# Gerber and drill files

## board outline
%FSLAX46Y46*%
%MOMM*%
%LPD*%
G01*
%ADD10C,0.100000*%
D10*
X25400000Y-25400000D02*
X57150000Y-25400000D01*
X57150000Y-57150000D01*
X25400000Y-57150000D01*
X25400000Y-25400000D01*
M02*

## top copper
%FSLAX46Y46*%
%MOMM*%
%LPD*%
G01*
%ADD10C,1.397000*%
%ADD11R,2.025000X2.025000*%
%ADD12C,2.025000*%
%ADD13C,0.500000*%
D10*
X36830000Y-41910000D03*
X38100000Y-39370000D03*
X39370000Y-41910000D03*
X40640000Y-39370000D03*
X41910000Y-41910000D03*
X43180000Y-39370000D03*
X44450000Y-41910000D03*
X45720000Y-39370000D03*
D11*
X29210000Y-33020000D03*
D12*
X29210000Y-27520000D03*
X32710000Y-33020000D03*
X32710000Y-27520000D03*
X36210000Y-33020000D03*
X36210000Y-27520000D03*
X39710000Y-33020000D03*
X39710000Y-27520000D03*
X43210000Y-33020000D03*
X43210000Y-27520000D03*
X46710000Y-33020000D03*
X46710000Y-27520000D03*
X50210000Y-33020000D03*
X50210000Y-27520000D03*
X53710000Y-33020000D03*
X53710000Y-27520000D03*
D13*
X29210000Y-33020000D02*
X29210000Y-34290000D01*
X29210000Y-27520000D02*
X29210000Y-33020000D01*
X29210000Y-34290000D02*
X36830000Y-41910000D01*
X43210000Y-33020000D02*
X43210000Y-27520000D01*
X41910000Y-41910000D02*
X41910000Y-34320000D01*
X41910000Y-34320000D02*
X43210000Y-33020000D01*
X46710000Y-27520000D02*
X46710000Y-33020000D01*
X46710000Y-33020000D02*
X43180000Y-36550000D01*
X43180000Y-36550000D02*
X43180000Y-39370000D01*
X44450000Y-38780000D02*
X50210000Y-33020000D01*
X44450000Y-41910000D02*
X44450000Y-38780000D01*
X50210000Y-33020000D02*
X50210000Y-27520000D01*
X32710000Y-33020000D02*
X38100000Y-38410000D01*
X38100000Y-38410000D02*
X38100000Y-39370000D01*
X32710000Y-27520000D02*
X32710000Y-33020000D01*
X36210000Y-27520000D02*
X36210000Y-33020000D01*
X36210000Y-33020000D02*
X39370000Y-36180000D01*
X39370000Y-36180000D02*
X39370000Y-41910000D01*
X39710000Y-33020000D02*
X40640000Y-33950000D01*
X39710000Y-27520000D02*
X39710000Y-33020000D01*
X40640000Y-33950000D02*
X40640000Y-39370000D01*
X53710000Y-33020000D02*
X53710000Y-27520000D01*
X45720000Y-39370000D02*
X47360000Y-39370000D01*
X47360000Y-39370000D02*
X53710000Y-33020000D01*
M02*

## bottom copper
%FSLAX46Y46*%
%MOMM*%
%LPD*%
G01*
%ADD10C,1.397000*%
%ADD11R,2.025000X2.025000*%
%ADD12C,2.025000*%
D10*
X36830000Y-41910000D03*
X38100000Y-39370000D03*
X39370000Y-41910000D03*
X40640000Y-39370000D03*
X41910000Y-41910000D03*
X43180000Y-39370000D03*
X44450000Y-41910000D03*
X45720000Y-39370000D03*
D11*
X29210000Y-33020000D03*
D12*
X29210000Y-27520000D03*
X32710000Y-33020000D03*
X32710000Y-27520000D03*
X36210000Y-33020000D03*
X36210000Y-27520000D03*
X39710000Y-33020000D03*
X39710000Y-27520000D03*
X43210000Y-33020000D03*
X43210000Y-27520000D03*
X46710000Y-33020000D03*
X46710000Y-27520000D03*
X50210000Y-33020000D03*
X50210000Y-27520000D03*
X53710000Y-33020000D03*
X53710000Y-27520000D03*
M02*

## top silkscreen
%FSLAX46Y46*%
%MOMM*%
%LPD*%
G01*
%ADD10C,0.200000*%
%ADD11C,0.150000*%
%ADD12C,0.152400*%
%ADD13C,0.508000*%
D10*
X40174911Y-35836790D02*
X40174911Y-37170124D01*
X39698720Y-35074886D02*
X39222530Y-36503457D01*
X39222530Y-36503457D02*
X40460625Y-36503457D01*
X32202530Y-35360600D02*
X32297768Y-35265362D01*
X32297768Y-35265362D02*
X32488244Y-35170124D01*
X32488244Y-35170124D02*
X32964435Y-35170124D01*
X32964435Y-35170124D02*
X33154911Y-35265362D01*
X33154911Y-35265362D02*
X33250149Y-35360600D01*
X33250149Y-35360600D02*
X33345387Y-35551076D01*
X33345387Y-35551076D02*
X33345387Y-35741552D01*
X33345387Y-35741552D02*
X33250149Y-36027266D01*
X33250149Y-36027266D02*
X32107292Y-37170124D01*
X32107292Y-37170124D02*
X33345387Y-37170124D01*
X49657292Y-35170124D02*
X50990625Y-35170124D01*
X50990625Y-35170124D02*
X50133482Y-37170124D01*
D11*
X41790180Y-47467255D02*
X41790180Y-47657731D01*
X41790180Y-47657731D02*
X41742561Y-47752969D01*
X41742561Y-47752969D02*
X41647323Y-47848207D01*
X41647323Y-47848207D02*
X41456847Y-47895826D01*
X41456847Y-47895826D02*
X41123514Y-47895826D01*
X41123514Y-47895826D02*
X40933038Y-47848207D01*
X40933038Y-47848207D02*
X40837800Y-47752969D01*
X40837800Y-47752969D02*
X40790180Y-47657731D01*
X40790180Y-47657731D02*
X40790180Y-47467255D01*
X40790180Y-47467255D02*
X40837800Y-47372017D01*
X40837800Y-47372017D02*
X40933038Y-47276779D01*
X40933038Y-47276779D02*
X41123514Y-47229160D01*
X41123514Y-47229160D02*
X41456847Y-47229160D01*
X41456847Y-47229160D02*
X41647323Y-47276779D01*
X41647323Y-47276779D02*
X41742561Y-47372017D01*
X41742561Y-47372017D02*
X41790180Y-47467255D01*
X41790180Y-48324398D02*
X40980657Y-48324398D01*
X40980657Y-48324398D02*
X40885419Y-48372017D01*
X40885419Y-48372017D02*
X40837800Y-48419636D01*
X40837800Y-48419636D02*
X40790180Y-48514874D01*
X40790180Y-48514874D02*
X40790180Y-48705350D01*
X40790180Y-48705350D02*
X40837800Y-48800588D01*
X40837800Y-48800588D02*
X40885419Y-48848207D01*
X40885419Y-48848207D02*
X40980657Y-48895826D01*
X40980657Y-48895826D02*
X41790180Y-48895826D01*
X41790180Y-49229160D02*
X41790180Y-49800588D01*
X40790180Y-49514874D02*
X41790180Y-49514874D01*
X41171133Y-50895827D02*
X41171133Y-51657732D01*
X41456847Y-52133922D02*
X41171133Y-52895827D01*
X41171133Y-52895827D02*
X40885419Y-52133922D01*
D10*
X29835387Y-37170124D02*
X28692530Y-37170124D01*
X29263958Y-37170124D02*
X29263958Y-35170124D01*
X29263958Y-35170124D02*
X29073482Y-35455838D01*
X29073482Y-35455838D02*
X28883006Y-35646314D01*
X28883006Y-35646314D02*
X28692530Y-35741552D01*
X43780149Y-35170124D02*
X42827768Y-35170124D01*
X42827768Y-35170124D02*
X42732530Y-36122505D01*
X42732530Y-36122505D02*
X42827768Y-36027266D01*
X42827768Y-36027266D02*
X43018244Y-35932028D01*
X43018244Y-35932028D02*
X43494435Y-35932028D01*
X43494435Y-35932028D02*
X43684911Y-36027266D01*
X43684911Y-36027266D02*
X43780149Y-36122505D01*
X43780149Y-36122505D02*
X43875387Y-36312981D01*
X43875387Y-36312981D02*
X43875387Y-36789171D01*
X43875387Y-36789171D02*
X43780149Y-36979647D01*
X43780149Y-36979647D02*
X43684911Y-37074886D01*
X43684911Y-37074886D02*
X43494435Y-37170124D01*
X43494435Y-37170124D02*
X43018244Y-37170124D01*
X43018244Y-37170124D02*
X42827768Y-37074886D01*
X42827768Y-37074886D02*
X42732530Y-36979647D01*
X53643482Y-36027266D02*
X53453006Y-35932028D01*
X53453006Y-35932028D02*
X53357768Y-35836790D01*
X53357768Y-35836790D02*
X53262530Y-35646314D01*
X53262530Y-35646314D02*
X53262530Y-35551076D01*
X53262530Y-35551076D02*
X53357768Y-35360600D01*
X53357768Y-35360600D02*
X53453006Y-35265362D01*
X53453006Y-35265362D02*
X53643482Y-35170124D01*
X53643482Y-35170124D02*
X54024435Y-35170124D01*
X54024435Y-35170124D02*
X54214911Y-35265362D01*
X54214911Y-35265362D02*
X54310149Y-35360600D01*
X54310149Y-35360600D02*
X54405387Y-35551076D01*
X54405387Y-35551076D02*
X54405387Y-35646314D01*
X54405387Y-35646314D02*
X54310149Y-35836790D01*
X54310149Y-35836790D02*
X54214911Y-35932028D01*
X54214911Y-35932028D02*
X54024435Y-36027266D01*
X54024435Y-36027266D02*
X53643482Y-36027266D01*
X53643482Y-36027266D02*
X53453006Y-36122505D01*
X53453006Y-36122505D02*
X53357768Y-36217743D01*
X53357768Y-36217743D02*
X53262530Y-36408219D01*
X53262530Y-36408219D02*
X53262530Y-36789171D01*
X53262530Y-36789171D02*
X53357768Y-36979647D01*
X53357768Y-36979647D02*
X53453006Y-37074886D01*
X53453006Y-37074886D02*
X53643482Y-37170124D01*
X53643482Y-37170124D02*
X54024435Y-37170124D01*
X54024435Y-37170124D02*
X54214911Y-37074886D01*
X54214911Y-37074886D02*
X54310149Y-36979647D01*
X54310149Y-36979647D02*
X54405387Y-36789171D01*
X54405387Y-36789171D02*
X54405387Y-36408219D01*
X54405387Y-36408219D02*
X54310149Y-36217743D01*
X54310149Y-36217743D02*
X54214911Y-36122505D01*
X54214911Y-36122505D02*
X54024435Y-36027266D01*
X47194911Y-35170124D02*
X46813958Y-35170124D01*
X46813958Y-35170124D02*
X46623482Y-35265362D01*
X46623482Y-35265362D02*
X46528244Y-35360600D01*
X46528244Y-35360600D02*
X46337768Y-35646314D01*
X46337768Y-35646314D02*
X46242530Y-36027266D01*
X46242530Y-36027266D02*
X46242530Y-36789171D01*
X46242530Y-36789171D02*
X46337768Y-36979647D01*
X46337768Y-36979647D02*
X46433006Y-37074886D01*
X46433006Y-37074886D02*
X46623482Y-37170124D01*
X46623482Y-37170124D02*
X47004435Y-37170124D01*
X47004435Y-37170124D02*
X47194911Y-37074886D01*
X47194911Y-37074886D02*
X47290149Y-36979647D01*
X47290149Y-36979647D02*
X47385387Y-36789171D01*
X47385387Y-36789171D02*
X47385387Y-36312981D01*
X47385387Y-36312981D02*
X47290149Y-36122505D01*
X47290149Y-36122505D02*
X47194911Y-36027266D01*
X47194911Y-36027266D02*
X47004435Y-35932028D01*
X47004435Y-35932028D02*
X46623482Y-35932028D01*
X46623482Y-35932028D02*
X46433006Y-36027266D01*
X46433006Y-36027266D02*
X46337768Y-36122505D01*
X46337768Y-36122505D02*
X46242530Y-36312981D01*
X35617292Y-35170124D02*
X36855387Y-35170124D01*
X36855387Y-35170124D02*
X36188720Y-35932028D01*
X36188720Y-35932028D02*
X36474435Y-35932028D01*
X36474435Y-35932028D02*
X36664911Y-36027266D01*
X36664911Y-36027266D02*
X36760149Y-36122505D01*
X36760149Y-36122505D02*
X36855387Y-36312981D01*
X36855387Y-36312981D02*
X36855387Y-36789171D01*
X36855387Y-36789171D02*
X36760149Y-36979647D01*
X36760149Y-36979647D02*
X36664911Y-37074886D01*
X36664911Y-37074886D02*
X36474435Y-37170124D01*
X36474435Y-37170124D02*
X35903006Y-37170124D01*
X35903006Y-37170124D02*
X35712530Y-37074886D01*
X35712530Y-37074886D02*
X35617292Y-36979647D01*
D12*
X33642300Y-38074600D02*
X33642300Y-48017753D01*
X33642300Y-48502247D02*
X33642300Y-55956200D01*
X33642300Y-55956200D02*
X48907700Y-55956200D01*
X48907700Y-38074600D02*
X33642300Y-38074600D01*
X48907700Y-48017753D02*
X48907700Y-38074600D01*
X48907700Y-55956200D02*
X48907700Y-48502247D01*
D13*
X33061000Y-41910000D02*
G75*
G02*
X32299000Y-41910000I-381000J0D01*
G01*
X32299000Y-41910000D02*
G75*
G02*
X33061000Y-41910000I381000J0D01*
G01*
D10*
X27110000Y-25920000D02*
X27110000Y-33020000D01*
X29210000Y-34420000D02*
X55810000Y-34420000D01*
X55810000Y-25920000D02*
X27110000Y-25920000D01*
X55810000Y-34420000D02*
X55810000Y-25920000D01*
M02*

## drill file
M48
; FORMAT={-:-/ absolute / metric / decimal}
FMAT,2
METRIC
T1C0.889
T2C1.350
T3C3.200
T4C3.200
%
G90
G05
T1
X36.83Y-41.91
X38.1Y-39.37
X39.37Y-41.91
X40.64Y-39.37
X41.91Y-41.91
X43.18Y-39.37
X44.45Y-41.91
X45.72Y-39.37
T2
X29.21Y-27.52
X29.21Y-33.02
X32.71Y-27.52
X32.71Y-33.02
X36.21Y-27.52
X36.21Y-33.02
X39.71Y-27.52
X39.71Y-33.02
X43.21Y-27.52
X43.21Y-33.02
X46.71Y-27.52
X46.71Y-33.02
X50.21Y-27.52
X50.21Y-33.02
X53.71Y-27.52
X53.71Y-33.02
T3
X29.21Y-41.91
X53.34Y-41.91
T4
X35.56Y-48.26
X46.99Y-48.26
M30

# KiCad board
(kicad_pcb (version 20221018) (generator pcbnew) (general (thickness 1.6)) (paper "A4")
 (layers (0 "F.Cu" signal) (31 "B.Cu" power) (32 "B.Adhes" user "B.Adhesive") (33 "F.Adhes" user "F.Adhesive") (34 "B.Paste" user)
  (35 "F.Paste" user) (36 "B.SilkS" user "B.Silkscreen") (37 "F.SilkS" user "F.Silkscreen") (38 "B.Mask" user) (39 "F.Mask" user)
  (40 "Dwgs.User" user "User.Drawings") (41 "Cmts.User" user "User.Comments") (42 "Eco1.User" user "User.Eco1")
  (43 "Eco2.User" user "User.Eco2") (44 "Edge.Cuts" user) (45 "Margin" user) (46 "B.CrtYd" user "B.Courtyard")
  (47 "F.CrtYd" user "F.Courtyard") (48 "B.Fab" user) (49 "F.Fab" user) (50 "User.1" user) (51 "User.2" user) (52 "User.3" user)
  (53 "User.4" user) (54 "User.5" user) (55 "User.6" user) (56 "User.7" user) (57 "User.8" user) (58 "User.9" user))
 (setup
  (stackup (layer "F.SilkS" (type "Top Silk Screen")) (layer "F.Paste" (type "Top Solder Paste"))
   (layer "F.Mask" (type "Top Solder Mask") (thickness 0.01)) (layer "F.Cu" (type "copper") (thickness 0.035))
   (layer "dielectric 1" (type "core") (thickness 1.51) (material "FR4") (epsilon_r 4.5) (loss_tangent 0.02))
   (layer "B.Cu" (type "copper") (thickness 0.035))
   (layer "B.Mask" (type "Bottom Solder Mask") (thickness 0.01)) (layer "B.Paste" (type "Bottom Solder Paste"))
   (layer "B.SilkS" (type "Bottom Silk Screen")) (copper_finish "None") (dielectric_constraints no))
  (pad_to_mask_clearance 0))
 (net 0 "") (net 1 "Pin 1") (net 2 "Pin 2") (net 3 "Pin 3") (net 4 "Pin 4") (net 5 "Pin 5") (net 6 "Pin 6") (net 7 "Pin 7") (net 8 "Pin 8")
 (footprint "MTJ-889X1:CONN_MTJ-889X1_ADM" (layer "F.Cu") (at 36.83 41.91)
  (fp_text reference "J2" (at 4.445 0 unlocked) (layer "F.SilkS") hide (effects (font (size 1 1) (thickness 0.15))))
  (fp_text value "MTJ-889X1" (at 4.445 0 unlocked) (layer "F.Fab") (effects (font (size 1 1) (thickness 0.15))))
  (fp_line (start -3.1877 -3.8354) (end -3.1877 6.107753) (stroke (width 0.1524) (type solid)) (layer "F.SilkS"))
  (fp_line (start -3.1877 6.592247) (end -3.1877 14.0462) (stroke (width 0.1524) (type solid)) (layer "F.SilkS"))
  (fp_line (start -3.1877 14.0462) (end 12.0777 14.0462) (stroke (width 0.1524) (type solid)) (layer "F.SilkS"))
  (fp_line (start 12.0777 -3.8354) (end -3.1877 -3.8354) (stroke (width 0.1524) (type solid)) (layer "F.SilkS"))
  (fp_line (start 12.0777 6.107753) (end 12.0777 -3.8354) (stroke (width 0.1524) (type solid)) (layer "F.SilkS"))
  (fp_line (start 12.0777 14.0462) (end 12.0777 6.592247) (stroke (width 0.1524) (type solid)) (layer "F.SilkS"))
  (fp_circle (center -4.15 0) (end -3.769 0) (stroke (width 0.508) (type solid)) (fill none) (layer "F.SilkS"))
  (pad "" np_thru_hole circle (at -1.27 6.35) (size 3.2004 3.2004) (drill 3.2004) (layers "F&B.Cu" "*.Mask"))
  (pad "" np_thru_hole circle (at 10.16 6.35) (size 3.2004 3.2004) (drill 3.2004) (layers "F&B.Cu" "*.Mask"))
  (pad "1" thru_hole circle (at 0 0) (size 1.397 1.397) (drill 0.889) (layers "*.Cu" "*.Mask") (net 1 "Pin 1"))
  (pad "2" thru_hole circle (at 1.27 -2.54) (size 1.397 1.397) (drill 0.889) (layers "*.Cu" "*.Mask") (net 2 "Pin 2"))
  (pad "3" thru_hole circle (at 2.54 0) (size 1.397 1.397) (drill 0.889) (layers "*.Cu" "*.Mask") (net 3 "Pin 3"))
  (pad "4" thru_hole circle (at 3.81 -2.54) (size 1.397 1.397) (drill 0.889) (layers "*.Cu" "*.Mask") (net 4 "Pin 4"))
  (pad "5" thru_hole circle (at 5.08 0) (size 1.397 1.397) (drill 0.889) (layers "*.Cu" "*.Mask") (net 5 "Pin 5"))
  (pad "6" thru_hole circle (at 6.35 -2.54) (size 1.397 1.397) (drill 0.889) (layers "*.Cu" "*.Mask") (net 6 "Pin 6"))
  (pad "7" thru_hole circle (at 7.62 0) (size 1.397 1.397) (drill 0.889) (layers "*.Cu" "*.Mask") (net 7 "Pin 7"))
  (pad "8" thru_hole circle (at 8.89 -2.54) (size 1.397 1.397) (drill 0.889) (layers "*.Cu" "*.Mask") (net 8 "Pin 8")))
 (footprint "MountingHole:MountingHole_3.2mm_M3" (layer "F.Cu") (at 53.34 41.91)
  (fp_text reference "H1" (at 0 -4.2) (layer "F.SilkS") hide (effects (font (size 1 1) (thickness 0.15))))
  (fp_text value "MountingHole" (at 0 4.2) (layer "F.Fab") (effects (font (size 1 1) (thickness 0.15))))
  (pad "" np_thru_hole circle (at 0 0) (size 3.2 3.2) (drill 3.2) (layers "*.Cu" "*.Mask")))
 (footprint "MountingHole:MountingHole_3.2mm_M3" (layer "F.Cu") (at 29.21 41.91)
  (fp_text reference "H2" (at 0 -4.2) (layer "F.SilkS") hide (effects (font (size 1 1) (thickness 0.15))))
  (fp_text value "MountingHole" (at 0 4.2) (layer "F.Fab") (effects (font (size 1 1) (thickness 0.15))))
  (pad "" np_thru_hole circle (at 0 0) (size 3.2 3.2) (drill 3.2) (layers "*.Cu" "*.Mask")))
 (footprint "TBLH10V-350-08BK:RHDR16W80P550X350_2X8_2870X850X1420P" (layer "F.Cu") (at 29.21 33.02)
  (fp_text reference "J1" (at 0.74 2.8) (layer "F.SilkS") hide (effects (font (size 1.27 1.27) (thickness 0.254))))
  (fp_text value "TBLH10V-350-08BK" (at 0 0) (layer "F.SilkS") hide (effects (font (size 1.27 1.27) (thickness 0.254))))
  (fp_line (start -2.1 -7.1) (end -2.1 0) (stroke (width 0.2) (type solid)) (layer "F.SilkS"))
  (fp_line (start 0 1.4) (end 26.6 1.4) (stroke (width 0.2) (type solid)) (layer "F.SilkS"))
  (fp_line (start 26.6 -7.1) (end -2.1 -7.1) (stroke (width 0.2) (type solid)) (layer "F.SilkS"))
  (fp_line (start 26.6 1.4) (end 26.6 -7.1) (stroke (width 0.2) (type solid)) (layer "F.SilkS"))
  (pad "1" thru_hole rect (at 0 0) (size 2.025 2.025) (drill 1.35) (layers "*.Cu" "*.Mask") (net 1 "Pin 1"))
  (pad "2" thru_hole circle (at 0 -5.5) (size 2.025 2.025) (drill 1.35) (layers "*.Cu" "*.Mask") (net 1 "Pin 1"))
  (pad "3" thru_hole circle (at 3.5 0) (size 2.025 2.025) (drill 1.35) (layers "*.Cu" "*.Mask") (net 2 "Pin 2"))
  (pad "4" thru_hole circle (at 3.5 -5.5) (size 2.025 2.025) (drill 1.35) (layers "*.Cu" "*.Mask") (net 2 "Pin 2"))
  (pad "5" thru_hole circle (at 7 0) (size 2.025 2.025) (drill 1.35) (layers "*.Cu" "*.Mask") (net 3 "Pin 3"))
  (pad "6" thru_hole circle (at 7 -5.5) (size 2.025 2.025) (drill 1.35) (layers "*.Cu" "*.Mask") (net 3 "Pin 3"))
  (pad "7" thru_hole circle (at 10.5 0) (size 2.025 2.025) (drill 1.35) (layers "*.Cu" "*.Mask") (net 4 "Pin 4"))
  (pad "8" thru_hole circle (at 10.5 -5.5) (size 2.025 2.025) (drill 1.35) (layers "*.Cu" "*.Mask") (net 4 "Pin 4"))
  (pad "9" thru_hole circle (at 14 0) (size 2.025 2.025) (drill 1.35) (layers "*.Cu" "*.Mask") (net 5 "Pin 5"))
  (pad "10" thru_hole circle (at 14 -5.5) (size 2.025 2.025) (drill 1.35) (layers "*.Cu" "*.Mask") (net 5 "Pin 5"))
  (pad "11" thru_hole circle (at 17.5 0) (size 2.025 2.025) (drill 1.35) (layers "*.Cu" "*.Mask") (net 6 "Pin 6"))
  (pad "12" thru_hole circle (at 17.5 -5.5) (size 2.025 2.025) (drill 1.35) (layers "*.Cu" "*.Mask") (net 6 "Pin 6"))
  (pad "13" thru_hole circle (at 21 0) (size 2.025 2.025) (drill 1.35) (layers "*.Cu" "*.Mask") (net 7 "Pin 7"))
  (pad "14" thru_hole circle (at 21 -5.5) (size 2.025 2.025) (drill 1.35) (layers "*.Cu" "*.Mask") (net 7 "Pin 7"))
  (pad "15" thru_hole circle (at 24.5 0) (size 2.025 2.025) (drill 1.35) (layers "*.Cu" "*.Mask") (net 8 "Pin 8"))
  (pad "16" thru_hole circle (at 24.5 -5.5) (size 2.025 2.025) (drill 1.35) (layers "*.Cu" "*.Mask") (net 8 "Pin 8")))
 (gr_rect (start 25.4 25.4) (end 57.15 57.15) (stroke (width 0.1) (type default)) (fill none) (layer "Edge.Cuts"))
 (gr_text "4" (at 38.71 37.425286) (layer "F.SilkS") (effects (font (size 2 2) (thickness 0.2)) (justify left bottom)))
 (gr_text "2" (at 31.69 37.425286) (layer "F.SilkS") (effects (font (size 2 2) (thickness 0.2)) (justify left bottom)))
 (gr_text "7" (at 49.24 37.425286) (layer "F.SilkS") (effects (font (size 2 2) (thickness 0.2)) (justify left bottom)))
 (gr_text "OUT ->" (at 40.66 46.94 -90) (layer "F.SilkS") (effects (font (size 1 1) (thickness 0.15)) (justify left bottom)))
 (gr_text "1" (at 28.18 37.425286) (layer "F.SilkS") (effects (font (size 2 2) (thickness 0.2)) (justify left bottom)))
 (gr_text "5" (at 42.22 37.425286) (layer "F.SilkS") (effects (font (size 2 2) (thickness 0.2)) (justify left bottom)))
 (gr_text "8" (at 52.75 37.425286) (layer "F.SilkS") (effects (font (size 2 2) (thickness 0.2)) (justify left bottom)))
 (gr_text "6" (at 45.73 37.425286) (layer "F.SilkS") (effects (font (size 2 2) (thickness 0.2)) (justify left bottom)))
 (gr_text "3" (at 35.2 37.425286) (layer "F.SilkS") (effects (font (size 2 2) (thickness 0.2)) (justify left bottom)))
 (segment (start 29.21 33.02) (end 29.21 34.29) (width 0.5) (layer "F.Cu") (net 1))
 (segment (start 29.21 27.52) (end 29.21 33.02) (width 0.5) (layer "F.Cu") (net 1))
 (segment (start 29.21 34.29) (end 36.83 41.91) (width 0.5) (layer "F.Cu") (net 1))
 (segment (start 43.21 33.02) (end 43.21 27.52) (width 0.5) (layer "F.Cu") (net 5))
 (segment (start 41.91 41.91) (end 41.91 34.32) (width 0.5) (layer "F.Cu") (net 5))
 (segment (start 41.91 34.32) (end 43.21 33.02) (width 0.5) (layer "F.Cu") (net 5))
 (segment (start 46.71 27.52) (end 46.71 33.02) (width 0.5) (layer "F.Cu") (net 6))
 (segment (start 46.71 33.02) (end 43.18 36.55) (width 0.5) (layer "F.Cu") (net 6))
 (segment (start 43.18 36.55) (end 43.18 39.37) (width 0.5) (layer "F.Cu") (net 6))
 (segment (start 44.45 38.78) (end 50.21 33.02) (width 0.5) (layer "F.Cu") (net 7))
 (segment (start 44.45 41.91) (end 44.45 38.78) (width 0.5) (layer "F.Cu") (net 7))
 (segment (start 50.21 33.02) (end 50.21 27.52) (width 0.5) (layer "F.Cu") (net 7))
 (segment (start 32.71 33.02) (end 38.1 38.41) (width 0.5) (layer "F.Cu") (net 2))
 (segment (start 38.1 38.41) (end 38.1 39.37) (width 0.5) (layer "F.Cu") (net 2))
 (segment (start 32.71 27.52) (end 32.71 33.02) (width 0.5) (layer "F.Cu") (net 2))
 (segment (start 36.21 27.52) (end 36.21 33.02) (width 0.5) (layer "F.Cu") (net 3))
 (segment (start 36.21 33.02) (end 39.37 36.18) (width 0.5) (layer "F.Cu") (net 3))
 (segment (start 39.37 36.18) (end 39.37 41.91) (width 0.5) (layer "F.Cu") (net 3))
 (segment (start 39.71 33.02) (end 40.64 33.95) (width 0.5) (layer "F.Cu") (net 4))
 (segment (start 39.71 27.52) (end 39.71 33.02) (width 0.5) (layer "F.Cu") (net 4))
 (segment (start 40.64 33.95) (end 40.64 39.37) (width 0.5) (layer "F.Cu") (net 4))
 (segment (start 53.71 33.02) (end 53.71 27.52) (width 0.5) (layer "F.Cu") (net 8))
 (segment (start 45.72 39.37) (end 47.36 39.37) (width 0.5) (layer "F.Cu") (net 8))
 (segment (start 47.36 39.37) (end 53.71 33.02) (width 0.5) (layer "F.Cu") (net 8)))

